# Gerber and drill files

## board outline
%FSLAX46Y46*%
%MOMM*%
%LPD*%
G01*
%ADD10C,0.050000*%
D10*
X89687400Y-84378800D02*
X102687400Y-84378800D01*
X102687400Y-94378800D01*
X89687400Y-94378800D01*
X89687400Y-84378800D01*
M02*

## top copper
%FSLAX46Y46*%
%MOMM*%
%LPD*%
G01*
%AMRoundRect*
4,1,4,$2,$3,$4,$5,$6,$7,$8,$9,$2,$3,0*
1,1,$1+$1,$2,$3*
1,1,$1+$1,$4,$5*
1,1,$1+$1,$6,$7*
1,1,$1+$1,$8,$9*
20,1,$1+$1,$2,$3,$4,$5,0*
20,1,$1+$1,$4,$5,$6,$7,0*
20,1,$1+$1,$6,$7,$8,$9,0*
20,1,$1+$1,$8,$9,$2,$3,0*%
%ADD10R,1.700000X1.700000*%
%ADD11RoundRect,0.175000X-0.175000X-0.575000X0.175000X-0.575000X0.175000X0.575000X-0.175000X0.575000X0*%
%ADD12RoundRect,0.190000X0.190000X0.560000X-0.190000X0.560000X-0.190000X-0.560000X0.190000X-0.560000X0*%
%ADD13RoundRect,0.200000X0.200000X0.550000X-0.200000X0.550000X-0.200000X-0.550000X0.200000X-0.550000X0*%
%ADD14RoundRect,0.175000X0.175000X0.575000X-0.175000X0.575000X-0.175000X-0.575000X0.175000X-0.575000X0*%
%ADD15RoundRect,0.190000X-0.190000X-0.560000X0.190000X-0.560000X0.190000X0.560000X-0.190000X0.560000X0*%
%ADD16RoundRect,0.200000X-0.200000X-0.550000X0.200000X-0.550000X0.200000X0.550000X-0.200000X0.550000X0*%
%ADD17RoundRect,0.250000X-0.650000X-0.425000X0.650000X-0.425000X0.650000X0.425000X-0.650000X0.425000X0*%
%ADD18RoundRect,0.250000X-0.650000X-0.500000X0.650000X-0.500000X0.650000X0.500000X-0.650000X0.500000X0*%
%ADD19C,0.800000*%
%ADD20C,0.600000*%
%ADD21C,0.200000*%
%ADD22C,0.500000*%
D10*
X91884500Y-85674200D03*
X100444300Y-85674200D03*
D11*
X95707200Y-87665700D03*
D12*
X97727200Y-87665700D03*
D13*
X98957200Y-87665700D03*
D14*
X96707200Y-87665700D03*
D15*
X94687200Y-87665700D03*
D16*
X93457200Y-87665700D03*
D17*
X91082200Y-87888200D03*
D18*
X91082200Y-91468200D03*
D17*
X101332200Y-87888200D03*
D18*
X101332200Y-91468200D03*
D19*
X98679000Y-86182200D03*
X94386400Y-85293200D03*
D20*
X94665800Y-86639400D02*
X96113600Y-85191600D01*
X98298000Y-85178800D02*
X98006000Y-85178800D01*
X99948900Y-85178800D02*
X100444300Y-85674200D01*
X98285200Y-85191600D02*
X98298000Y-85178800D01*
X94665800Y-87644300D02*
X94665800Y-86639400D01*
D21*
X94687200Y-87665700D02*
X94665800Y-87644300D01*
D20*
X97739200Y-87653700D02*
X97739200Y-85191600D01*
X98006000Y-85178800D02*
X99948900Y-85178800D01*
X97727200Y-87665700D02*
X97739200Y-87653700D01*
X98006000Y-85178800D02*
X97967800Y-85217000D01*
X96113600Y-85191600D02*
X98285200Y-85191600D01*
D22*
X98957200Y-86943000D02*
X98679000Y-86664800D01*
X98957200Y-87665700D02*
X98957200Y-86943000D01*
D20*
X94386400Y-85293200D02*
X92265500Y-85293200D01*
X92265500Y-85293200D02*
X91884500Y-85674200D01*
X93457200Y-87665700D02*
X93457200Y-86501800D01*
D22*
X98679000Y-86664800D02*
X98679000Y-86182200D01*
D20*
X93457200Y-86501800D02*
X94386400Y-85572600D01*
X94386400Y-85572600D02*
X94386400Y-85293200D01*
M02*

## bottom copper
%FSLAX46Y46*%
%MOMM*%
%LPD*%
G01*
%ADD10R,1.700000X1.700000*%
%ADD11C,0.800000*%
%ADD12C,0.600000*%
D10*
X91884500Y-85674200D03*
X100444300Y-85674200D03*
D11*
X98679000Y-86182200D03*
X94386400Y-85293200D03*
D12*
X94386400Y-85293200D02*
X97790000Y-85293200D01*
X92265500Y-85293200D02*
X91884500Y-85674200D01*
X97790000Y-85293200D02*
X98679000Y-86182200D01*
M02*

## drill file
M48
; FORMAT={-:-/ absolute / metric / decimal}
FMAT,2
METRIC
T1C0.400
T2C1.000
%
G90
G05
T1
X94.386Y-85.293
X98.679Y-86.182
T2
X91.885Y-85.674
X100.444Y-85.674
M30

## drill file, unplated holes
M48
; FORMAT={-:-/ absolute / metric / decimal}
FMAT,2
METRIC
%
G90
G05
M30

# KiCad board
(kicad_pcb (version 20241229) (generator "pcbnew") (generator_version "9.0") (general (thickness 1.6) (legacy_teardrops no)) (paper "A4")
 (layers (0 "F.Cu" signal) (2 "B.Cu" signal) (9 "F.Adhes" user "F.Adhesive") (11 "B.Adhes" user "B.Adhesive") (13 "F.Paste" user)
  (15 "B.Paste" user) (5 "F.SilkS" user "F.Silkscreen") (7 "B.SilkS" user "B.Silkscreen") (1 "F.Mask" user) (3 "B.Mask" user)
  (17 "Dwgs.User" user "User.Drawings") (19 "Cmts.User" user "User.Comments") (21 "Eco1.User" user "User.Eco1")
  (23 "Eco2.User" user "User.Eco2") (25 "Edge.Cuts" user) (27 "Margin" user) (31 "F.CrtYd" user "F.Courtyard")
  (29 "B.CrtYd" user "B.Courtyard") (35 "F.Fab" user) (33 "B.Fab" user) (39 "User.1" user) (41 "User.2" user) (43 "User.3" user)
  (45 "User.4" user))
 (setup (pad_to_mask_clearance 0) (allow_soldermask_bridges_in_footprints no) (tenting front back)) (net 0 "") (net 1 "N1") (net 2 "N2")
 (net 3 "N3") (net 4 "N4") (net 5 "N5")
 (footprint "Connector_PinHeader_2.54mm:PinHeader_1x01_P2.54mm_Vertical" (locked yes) (layer "F.Cu") (at 91.8845 85.6742)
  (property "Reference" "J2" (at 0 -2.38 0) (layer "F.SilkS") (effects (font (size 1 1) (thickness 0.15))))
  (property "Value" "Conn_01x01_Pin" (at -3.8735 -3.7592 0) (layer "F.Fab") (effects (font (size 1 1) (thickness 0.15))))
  (pad "1" thru_hole rect (at 0 0) (size 1.7 1.7) (drill 1) (layers "*.Cu" "*.Mask") (remove_unused_layers no) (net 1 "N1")))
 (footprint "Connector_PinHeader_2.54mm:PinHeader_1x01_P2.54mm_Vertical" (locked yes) (layer "F.Cu") (at 100.4443 85.6742)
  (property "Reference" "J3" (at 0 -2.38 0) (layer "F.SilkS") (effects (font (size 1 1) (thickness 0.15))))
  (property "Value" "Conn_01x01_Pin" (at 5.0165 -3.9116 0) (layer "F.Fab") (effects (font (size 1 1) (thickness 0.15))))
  (pad "1" thru_hole rect (at 0 0) (size 1.7 1.7) (drill 1) (layers "*.Cu" "*.Mask") (remove_unused_layers no) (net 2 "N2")))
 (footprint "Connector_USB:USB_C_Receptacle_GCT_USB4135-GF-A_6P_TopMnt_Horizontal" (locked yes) (layer "F.Cu") (at 96.2072 90.8657)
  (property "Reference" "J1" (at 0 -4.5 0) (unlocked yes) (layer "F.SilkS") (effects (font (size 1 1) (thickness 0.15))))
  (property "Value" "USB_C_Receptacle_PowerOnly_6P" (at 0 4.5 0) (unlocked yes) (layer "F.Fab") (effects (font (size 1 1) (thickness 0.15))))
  (pad "A5" smd roundrect (at -0.5 -3.2) (size 0.7 1.5) (layers "F.Cu" "F.Mask" "F.Paste") (roundrect_rratio 0.25) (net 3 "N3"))
  (pad "A9" smd roundrect (at 1.52 -3.2 180) (size 0.76 1.5) (layers "F.Cu" "F.Mask" "F.Paste") (roundrect_rratio 0.25) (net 2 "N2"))
  (pad "A12" smd roundrect (at 2.75 -3.2 180) (size 0.8 1.5) (layers "F.Cu" "F.Mask" "F.Paste") (roundrect_rratio 0.25) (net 1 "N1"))
  (pad "B5" smd roundrect (at 0.5 -3.2 180) (size 0.7 1.5) (layers "F.Cu" "F.Mask" "F.Paste") (roundrect_rratio 0.25) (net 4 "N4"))
  (pad "B9" smd roundrect (at -1.52 -3.2) (size 0.76 1.5) (layers "F.Cu" "F.Mask" "F.Paste") (roundrect_rratio 0.25) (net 2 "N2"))
  (pad "B12" smd roundrect (at -2.75 -3.2) (size 0.8 1.5) (layers "F.Cu" "F.Mask" "F.Paste") (roundrect_rratio 0.25) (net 1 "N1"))
  (pad "S1" smd roundrect (at -5.125 -2.9775) (size 1.8 1.35) (layers "F.Cu" "F.Mask" "F.Paste") (roundrect_rratio 0.1851851852)
   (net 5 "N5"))
  (pad "S1" smd roundrect (at -5.125 0.6025) (size 1.8 1.5) (layers "F.Cu" "F.Mask" "F.Paste") (roundrect_rratio 0.1666666667) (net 5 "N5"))
  (pad "S1" smd roundrect (at 5.125 -2.9775) (size 1.8 1.35) (layers "F.Cu" "F.Mask" "F.Paste") (roundrect_rratio 0.1851851852) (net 5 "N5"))
  (pad "S1" smd roundrect (at 5.125 0.6025) (size 1.8 1.5) (layers "F.Cu" "F.Mask" "F.Paste") (roundrect_rratio 0.1666666667) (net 5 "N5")))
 (gr_rect (start 89.6874 84.3788) (end 102.6874 94.3788) (stroke (width 0.05) (type solid)) (fill no) (layer "Edge.Cuts"))
 (segment (start 94.6658 86.6394) (end 96.1136 85.1916) (width 0.6) (layer "F.Cu") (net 2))
 (segment (start 98.298 85.1788) (end 98.006 85.1788) (width 0.6) (layer "F.Cu") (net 2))
 (segment (start 99.9489 85.1788) (end 100.4443 85.6742) (width 0.6) (layer "F.Cu") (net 2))
 (segment (start 98.2852 85.1916) (end 98.298 85.1788) (width 0.6) (layer "F.Cu") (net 2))
 (segment (start 94.6658 87.6443) (end 94.6658 86.6394) (width 0.6) (layer "F.Cu") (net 2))
 (segment (start 94.6872 87.6657) (end 94.6658 87.6443) (width 0.2) (layer "F.Cu") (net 2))
 (segment (start 97.7392 87.6537) (end 97.7392 85.1916) (width 0.6) (layer "F.Cu") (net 2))
 (segment (start 98.006 85.1788) (end 99.9489 85.1788) (width 0.6) (layer "F.Cu") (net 2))
 (segment (start 97.7272 87.6657) (end 97.7392 87.6537) (width 0.6) (layer "F.Cu") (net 2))
 (segment (start 98.006 85.1788) (end 97.9678 85.217) (width 0.6) (layer "F.Cu") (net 2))
 (segment (start 96.1136 85.1916) (end 98.2852 85.1916) (width 0.6) (layer "F.Cu") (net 2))
 (segment (start 98.9572 86.943) (end 98.679 86.6648) (width 0.5) (layer "F.Cu") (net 1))
 (segment (start 98.9572 87.6657) (end 98.9572 86.943) (width 0.5) (layer "F.Cu") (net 1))
 (segment (start 94.3864 85.2932) (end 92.2655 85.2932) (width 0.6) (layer "F.Cu") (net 1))
 (segment (start 92.2655 85.2932) (end 91.8845 85.6742) (width 0.6) (layer "F.Cu") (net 1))
 (segment (start 93.4572 87.6657) (end 93.4572 86.5018) (width 0.6) (layer "F.Cu") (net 1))
 (segment (start 98.679 86.6648) (end 98.679 86.1822) (width 0.5) (layer "F.Cu") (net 1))
 (segment (start 93.4572 86.5018) (end 94.3864 85.5726) (width 0.6) (layer "F.Cu") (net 1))
 (segment (start 94.3864 85.5726) (end 94.3864 85.2932) (width 0.6) (layer "F.Cu") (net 1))
 (via (at 98.679 86.1822) (size 0.8) (drill 0.4) (layers "F.Cu" "B.Cu") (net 1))
 (via (at 94.3864 85.2932) (size 0.8) (drill 0.4) (layers "F.Cu" "B.Cu") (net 1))
 (segment (start 94.3864 85.2932) (end 97.79 85.2932) (width 0.6) (layer "B.Cu") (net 1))
 (segment (start 92.2655 85.2932) (end 91.8845 85.6742) (width 0.6) (layer "B.Cu") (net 1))
 (segment (start 97.79 85.2932) (end 98.679 86.1822) (width 0.6) (layer "B.Cu") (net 1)))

